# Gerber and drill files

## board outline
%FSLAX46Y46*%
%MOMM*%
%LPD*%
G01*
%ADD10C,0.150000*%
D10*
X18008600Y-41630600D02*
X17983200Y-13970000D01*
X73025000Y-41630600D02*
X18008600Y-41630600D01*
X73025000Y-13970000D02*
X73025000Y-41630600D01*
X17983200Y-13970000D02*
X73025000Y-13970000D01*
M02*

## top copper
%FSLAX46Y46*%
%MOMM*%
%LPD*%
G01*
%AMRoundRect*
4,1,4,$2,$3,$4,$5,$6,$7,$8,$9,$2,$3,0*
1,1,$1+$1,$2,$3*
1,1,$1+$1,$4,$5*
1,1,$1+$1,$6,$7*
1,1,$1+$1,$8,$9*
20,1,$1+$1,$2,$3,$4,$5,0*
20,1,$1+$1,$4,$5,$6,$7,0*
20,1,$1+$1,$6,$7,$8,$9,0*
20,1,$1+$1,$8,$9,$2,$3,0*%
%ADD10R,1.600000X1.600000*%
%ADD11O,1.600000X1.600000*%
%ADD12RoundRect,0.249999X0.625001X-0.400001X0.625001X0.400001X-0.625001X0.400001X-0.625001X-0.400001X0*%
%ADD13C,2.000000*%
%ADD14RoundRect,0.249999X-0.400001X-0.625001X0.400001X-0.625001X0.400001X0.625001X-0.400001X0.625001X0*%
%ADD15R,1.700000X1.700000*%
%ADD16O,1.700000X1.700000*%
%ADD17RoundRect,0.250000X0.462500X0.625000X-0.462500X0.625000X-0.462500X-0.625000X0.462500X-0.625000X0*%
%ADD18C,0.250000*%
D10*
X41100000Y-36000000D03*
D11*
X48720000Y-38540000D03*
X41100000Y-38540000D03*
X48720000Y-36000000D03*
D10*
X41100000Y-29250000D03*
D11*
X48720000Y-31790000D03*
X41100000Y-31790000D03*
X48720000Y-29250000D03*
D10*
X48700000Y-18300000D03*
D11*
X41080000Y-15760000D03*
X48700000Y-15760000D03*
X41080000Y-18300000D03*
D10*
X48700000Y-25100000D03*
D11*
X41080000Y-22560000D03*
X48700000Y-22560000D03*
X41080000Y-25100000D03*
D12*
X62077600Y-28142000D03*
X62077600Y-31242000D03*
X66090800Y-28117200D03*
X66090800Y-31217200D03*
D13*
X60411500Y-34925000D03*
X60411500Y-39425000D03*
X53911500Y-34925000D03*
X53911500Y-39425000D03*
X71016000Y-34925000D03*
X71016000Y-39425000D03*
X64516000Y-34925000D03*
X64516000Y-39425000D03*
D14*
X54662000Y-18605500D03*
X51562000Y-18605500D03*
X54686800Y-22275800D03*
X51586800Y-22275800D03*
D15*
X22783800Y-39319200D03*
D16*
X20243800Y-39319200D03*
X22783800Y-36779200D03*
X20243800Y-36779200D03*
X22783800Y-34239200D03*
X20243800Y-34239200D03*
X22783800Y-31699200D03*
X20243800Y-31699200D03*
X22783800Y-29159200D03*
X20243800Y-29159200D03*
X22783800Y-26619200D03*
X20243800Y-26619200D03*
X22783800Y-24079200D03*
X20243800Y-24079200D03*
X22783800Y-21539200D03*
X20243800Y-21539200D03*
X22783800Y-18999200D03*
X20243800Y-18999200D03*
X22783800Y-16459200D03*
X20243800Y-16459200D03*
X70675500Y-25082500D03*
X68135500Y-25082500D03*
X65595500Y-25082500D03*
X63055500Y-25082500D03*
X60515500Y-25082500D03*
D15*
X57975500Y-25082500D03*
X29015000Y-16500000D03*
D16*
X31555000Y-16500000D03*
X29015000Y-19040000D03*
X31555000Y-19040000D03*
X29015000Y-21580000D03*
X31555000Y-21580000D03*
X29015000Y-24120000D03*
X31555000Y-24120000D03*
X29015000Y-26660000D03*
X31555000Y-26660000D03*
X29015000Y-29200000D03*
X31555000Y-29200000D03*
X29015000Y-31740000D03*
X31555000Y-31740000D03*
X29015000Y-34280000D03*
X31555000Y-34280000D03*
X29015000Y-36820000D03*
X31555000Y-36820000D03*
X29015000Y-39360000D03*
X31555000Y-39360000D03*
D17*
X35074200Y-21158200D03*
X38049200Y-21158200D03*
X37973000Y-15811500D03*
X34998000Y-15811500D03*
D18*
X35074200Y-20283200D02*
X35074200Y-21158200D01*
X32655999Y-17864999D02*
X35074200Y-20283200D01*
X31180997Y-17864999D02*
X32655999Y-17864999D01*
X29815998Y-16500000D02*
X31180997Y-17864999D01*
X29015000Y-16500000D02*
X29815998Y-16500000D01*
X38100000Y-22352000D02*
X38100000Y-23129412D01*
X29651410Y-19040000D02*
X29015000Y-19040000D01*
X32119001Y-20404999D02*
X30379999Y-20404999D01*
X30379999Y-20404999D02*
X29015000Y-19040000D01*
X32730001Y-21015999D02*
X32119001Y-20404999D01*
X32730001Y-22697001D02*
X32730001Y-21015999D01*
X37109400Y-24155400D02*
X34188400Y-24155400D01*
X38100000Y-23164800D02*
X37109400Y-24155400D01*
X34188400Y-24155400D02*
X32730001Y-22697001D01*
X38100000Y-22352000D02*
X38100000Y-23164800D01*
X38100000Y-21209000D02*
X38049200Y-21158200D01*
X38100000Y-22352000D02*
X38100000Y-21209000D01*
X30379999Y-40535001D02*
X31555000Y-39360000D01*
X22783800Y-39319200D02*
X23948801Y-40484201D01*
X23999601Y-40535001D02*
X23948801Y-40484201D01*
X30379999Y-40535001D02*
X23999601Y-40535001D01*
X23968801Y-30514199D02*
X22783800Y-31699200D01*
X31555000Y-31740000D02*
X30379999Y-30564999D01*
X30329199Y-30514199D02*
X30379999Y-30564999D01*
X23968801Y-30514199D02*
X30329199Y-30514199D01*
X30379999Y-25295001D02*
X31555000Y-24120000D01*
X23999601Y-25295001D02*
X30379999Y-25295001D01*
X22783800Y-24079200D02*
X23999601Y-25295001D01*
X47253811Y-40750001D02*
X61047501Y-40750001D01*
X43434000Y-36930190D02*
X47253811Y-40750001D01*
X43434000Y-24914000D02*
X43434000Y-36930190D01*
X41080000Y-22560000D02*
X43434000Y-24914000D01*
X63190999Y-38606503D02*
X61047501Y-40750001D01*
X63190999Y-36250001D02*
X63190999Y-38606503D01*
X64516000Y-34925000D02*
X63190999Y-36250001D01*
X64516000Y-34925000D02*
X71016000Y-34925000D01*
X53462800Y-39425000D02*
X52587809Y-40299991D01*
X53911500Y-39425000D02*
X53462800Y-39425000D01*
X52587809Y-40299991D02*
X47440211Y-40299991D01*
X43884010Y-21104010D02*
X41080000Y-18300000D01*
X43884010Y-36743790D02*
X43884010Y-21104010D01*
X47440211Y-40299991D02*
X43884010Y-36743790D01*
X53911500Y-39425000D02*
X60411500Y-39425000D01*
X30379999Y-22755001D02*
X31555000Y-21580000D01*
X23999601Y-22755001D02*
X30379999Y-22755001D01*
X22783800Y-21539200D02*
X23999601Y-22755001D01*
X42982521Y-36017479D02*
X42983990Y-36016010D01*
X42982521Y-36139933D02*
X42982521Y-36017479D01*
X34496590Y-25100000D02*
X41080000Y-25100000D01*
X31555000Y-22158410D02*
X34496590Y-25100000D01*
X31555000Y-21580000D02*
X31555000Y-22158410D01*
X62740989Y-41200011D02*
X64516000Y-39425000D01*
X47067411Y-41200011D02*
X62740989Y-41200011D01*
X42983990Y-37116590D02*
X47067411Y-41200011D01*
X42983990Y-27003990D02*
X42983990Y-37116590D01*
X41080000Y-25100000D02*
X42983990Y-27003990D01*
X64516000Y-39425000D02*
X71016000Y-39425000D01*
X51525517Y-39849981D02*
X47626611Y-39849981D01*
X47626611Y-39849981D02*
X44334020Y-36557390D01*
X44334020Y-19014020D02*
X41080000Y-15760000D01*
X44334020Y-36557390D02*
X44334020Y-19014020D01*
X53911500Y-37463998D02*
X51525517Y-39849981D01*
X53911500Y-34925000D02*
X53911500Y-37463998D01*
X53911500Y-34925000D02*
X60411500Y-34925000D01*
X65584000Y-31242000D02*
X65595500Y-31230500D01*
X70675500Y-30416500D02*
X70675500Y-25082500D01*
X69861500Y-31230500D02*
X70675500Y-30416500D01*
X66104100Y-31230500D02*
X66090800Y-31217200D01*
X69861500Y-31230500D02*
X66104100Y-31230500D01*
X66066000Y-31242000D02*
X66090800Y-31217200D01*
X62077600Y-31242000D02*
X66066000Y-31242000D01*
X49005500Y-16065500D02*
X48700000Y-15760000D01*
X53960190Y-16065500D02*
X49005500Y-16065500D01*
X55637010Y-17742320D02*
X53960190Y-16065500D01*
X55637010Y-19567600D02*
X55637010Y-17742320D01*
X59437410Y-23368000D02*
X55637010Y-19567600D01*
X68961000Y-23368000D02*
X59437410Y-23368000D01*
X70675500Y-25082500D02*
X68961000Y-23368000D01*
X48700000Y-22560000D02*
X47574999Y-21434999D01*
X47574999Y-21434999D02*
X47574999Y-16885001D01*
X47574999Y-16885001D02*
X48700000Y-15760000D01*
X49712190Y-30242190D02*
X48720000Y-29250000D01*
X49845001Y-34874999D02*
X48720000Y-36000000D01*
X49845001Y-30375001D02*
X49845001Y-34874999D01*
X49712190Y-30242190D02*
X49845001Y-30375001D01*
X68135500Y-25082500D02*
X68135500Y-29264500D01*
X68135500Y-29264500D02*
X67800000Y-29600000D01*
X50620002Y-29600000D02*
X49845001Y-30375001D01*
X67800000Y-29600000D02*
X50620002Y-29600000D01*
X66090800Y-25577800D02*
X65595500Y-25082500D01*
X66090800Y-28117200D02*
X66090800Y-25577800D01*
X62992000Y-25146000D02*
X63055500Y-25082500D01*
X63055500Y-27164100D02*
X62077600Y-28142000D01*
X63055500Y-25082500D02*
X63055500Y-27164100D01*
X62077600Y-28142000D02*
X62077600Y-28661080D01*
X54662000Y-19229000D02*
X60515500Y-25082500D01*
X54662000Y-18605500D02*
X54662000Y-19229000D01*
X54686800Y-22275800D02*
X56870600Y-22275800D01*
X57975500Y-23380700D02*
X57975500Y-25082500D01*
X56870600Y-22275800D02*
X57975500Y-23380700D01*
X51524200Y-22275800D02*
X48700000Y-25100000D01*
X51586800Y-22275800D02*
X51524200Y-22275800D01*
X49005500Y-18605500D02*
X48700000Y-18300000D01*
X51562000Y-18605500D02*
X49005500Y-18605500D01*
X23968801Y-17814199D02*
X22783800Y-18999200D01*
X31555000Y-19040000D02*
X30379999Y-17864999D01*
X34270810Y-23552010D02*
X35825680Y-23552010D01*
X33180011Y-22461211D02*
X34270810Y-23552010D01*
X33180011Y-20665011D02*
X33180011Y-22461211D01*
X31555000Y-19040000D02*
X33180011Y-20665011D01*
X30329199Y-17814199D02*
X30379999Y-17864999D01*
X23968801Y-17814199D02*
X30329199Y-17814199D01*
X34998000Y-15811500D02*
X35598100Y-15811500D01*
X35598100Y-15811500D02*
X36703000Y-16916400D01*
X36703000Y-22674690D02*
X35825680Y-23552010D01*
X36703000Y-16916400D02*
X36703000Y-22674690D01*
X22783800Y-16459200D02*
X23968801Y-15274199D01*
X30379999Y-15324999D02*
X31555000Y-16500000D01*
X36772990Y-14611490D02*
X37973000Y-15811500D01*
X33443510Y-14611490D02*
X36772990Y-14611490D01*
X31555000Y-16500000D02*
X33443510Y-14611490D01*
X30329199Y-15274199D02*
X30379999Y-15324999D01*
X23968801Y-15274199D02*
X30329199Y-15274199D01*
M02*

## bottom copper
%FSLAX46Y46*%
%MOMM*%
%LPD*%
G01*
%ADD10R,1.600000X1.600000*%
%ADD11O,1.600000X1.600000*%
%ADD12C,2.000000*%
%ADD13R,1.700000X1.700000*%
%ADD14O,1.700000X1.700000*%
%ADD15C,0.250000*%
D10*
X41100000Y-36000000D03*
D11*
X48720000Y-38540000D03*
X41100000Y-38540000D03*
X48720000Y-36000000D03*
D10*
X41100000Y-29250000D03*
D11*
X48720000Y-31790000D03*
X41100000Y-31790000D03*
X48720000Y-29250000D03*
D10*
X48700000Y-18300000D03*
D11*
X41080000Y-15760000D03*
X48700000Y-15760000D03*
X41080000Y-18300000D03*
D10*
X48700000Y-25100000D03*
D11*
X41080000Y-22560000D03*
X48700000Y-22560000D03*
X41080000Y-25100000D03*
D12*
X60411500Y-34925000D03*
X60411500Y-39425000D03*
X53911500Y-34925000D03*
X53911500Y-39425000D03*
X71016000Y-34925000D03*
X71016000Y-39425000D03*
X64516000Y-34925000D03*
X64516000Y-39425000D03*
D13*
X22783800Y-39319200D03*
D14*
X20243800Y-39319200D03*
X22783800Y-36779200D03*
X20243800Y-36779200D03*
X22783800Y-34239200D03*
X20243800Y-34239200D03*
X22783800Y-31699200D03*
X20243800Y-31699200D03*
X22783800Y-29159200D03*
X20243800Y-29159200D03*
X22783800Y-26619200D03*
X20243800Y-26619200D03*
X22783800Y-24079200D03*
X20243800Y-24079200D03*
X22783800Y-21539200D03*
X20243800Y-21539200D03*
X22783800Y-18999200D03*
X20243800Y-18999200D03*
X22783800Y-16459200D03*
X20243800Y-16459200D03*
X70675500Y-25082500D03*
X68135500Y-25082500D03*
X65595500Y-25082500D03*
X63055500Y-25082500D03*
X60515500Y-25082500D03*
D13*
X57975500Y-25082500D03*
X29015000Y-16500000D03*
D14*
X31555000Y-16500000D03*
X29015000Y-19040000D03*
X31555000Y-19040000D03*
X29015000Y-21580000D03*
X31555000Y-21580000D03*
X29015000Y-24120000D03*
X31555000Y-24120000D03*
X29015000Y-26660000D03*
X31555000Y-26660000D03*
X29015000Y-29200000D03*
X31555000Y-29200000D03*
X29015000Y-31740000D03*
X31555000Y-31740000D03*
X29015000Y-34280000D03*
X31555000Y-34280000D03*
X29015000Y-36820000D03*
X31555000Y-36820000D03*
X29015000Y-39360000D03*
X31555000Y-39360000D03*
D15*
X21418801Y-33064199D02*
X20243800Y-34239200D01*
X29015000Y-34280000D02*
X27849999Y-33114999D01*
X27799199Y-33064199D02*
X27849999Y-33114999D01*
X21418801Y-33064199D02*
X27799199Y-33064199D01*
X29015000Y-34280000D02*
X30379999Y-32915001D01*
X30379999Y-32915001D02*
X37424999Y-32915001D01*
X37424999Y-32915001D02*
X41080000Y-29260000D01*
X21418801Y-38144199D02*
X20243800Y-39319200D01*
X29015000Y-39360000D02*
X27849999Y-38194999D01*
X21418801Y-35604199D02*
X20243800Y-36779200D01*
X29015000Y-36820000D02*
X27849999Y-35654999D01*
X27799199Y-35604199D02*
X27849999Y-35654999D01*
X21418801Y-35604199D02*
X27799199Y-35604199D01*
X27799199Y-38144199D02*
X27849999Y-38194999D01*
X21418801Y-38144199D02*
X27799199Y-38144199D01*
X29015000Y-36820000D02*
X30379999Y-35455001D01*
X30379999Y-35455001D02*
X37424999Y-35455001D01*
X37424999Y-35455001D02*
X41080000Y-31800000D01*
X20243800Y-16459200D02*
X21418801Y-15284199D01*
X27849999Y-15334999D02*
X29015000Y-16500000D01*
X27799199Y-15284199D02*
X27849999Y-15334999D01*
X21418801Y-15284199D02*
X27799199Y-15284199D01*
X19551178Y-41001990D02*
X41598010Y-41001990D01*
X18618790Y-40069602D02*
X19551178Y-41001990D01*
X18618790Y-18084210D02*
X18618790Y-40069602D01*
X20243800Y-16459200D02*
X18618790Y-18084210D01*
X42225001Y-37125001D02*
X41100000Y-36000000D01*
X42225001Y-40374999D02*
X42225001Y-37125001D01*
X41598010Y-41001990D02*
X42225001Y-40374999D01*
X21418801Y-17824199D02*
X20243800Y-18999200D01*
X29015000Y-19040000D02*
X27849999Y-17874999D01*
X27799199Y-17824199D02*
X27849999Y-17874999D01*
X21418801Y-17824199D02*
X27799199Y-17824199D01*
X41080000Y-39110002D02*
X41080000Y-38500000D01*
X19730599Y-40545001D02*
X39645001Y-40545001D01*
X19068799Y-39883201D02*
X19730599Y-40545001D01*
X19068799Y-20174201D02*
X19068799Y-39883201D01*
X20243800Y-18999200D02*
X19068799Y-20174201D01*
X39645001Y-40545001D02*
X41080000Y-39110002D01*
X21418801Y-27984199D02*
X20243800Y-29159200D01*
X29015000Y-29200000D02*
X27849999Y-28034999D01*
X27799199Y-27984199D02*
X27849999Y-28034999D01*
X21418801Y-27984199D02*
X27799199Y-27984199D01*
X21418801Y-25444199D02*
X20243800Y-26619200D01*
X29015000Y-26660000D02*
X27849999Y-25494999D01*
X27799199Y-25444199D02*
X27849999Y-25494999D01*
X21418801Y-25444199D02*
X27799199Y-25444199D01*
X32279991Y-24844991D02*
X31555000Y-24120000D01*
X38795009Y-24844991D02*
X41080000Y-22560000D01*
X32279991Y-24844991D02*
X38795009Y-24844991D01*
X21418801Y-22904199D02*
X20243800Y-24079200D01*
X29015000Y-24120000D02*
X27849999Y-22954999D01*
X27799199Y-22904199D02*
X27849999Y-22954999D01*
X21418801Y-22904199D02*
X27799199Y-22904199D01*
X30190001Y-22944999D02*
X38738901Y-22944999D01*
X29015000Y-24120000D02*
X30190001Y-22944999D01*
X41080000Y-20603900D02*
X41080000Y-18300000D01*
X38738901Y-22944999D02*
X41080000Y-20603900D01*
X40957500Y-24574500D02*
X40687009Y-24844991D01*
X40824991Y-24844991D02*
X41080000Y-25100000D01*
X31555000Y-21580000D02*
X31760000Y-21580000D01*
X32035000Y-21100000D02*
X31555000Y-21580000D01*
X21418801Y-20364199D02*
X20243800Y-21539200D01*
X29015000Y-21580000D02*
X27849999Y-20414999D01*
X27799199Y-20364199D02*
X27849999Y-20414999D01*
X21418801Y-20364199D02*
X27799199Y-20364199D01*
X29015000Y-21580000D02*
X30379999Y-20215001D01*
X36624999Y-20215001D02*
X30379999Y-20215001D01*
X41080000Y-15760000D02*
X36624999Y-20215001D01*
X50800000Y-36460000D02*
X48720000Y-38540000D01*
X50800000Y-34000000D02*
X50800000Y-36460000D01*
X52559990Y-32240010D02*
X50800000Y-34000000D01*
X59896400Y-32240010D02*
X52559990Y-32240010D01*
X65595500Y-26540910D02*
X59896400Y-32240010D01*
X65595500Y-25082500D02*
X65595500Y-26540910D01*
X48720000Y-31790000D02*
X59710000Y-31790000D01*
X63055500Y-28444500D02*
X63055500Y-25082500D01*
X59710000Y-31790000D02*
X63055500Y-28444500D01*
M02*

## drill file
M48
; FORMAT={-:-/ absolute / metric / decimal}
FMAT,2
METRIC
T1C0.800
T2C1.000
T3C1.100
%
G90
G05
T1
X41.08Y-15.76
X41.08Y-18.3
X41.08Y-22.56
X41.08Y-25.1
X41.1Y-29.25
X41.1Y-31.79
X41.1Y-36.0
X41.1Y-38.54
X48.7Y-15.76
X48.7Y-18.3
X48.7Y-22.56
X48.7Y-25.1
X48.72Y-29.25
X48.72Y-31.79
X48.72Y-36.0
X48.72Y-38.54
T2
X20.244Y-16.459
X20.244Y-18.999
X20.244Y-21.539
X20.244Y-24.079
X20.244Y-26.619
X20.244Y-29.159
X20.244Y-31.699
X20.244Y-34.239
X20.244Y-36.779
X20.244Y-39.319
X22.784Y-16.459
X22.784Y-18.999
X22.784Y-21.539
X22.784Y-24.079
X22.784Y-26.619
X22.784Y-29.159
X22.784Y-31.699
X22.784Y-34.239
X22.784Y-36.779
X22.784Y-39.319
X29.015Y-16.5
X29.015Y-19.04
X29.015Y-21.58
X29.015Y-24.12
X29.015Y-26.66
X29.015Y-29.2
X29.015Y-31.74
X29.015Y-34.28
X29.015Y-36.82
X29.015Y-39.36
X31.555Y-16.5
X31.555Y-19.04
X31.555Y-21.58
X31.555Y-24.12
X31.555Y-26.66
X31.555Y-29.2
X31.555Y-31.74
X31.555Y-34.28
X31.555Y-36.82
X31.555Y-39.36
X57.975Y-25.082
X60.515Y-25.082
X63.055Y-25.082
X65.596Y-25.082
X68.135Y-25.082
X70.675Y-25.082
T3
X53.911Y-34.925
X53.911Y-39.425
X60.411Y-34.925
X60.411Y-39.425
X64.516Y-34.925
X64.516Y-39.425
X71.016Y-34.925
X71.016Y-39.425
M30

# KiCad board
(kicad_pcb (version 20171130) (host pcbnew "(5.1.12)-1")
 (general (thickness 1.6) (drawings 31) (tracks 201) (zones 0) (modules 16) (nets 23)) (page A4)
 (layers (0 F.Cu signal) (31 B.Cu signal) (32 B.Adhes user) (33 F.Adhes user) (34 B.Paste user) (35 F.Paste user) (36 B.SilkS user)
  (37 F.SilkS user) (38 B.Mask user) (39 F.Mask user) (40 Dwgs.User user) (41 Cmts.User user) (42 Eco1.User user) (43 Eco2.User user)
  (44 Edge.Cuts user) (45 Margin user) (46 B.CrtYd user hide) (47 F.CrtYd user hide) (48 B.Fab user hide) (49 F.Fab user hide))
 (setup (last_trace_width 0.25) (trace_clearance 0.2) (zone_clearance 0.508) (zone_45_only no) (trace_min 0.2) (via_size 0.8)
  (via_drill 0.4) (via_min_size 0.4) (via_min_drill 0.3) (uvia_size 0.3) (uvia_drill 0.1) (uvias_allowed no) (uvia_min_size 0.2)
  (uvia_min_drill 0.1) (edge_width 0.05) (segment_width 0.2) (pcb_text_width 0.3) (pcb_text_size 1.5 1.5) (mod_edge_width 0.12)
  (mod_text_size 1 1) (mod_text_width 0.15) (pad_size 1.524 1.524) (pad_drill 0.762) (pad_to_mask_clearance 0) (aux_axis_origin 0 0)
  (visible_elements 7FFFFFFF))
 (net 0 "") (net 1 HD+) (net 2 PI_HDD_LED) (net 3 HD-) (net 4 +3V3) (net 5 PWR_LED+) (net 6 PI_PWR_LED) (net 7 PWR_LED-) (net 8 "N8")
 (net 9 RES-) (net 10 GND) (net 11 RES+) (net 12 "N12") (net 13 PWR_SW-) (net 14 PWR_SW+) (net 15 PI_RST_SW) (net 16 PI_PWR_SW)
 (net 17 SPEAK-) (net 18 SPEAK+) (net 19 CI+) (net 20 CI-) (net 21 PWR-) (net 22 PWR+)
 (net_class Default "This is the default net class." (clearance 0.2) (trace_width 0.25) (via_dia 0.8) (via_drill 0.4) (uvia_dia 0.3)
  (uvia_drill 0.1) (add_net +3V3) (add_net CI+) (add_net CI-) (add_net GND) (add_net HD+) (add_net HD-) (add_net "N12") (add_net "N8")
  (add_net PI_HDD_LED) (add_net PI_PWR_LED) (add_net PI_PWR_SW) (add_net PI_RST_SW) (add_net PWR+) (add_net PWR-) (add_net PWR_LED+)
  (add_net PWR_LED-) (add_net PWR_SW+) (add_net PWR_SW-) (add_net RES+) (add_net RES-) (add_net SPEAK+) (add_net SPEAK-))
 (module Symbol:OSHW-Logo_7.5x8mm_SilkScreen (layer F.Cu) (at 54.4 29.5 270)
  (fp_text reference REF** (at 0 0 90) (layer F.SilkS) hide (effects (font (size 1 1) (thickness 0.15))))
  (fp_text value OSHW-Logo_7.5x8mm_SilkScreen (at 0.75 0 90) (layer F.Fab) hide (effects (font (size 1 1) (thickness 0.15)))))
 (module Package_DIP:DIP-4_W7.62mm (layer F.Cu) (at 41.1 36)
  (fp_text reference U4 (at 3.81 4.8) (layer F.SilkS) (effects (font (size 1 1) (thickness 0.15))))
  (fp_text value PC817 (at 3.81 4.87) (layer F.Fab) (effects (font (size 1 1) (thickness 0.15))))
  (pad 1 thru_hole rect (at 0 0) (size 1.6 1.6) (drill 0.8) (layers *.Cu *.Mask) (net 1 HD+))
  (pad 3 thru_hole oval (at 7.62 2.54) (size 1.6 1.6) (drill 0.8) (layers *.Cu *.Mask) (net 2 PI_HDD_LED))
  (pad 2 thru_hole oval (at 0 2.54) (size 1.6 1.6) (drill 0.8) (layers *.Cu *.Mask) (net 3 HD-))
  (pad 4 thru_hole oval (at 7.62 0) (size 1.6 1.6) (drill 0.8) (layers *.Cu *.Mask) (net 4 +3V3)))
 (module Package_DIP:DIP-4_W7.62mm (layer F.Cu) (at 41.1 29.25)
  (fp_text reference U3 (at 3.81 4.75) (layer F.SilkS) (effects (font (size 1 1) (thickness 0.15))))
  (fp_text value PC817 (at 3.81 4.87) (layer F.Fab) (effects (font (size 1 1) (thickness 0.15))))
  (pad 1 thru_hole rect (at 0 0) (size 1.6 1.6) (drill 0.8) (layers *.Cu *.Mask) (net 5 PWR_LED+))
  (pad 3 thru_hole oval (at 7.62 2.54) (size 1.6 1.6) (drill 0.8) (layers *.Cu *.Mask) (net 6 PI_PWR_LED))
  (pad 2 thru_hole oval (at 0 2.54) (size 1.6 1.6) (drill 0.8) (layers *.Cu *.Mask) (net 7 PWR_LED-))
  (pad 4 thru_hole oval (at 7.62 0) (size 1.6 1.6) (drill 0.8) (layers *.Cu *.Mask) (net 4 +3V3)))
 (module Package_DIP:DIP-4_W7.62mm (layer F.Cu) (at 48.7 18.3 180)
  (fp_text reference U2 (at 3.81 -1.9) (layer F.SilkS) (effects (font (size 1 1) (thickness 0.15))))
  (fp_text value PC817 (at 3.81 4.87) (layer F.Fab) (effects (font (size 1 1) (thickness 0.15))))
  (pad 1 thru_hole rect (at 0 0 180) (size 1.6 1.6) (drill 0.8) (layers *.Cu *.Mask) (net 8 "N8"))
  (pad 3 thru_hole oval (at 7.62 2.54 180) (size 1.6 1.6) (drill 0.8) (layers *.Cu *.Mask) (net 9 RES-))
  (pad 2 thru_hole oval (at 0 2.54 180) (size 1.6 1.6) (drill 0.8) (layers *.Cu *.Mask) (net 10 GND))
  (pad 4 thru_hole oval (at 7.62 0 180) (size 1.6 1.6) (drill 0.8) (layers *.Cu *.Mask) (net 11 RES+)))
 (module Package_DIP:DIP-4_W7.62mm (layer F.Cu) (at 48.7 25.1 180)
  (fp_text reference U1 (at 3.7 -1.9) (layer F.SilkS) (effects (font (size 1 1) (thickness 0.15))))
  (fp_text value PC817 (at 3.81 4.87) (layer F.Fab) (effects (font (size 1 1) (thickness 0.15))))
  (pad 1 thru_hole rect (at 0 0 180) (size 1.6 1.6) (drill 0.8) (layers *.Cu *.Mask) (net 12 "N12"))
  (pad 3 thru_hole oval (at 7.62 2.54 180) (size 1.6 1.6) (drill 0.8) (layers *.Cu *.Mask) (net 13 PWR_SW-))
  (pad 2 thru_hole oval (at 0 2.54 180) (size 1.6 1.6) (drill 0.8) (layers *.Cu *.Mask) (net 10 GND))
  (pad 4 thru_hole oval (at 7.62 0 180) (size 1.6 1.6) (drill 0.8) (layers *.Cu *.Mask) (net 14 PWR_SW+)))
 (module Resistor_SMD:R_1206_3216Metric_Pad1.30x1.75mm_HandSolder (layer F.Cu) (at 62.0776 29.692 90)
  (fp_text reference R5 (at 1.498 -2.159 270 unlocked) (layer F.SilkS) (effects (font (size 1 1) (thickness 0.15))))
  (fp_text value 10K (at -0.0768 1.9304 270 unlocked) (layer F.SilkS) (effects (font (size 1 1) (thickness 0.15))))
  (pad 2 smd roundrect (at 1.55 0 90) (size 1.3 1.75) (layers F.Cu F.Paste F.Mask) (roundrect_rratio 0.1923069230769231) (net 6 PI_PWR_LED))
  (pad 1 smd roundrect (at -1.55 0 90) (size 1.3 1.75) (layers F.Cu F.Paste F.Mask) (roundrect_rratio 0.1923069230769231) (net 10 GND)))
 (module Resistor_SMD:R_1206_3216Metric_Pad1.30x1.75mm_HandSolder (layer F.Cu) (at 66.0908 29.6672 90)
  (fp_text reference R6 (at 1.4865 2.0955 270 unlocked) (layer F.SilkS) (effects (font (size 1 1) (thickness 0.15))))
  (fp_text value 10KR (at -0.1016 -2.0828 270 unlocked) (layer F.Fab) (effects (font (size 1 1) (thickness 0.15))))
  (pad 2 smd roundrect (at 1.55 0 90) (size 1.3 1.75) (layers F.Cu F.Paste F.Mask) (roundrect_rratio 0.1923069230769231) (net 2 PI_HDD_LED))
  (pad 1 smd roundrect (at -1.55 0 90) (size 1.3 1.75) (layers F.Cu F.Paste F.Mask) (roundrect_rratio 0.1923069230769231) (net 10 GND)))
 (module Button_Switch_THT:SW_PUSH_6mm (layer F.Cu) (at 53.9115 34.925)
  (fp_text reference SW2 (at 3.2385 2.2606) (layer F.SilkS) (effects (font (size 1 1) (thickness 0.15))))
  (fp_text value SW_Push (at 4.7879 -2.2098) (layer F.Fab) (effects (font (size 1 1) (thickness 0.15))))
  (pad 1 thru_hole circle (at 6.5 0 90) (size 2 2) (drill 1.1) (layers *.Cu *.Mask) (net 9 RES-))
  (pad 2 thru_hole circle (at 6.5 4.5 90) (size 2 2) (drill 1.1) (layers *.Cu *.Mask) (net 11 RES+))
  (pad 1 thru_hole circle (at 0 0 90) (size 2 2) (drill 1.1) (layers *.Cu *.Mask) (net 9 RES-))
  (pad 2 thru_hole circle (at 0 4.5 90) (size 2 2) (drill 1.1) (layers *.Cu *.Mask) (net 11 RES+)))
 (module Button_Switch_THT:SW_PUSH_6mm (layer F.Cu) (at 64.516 34.925)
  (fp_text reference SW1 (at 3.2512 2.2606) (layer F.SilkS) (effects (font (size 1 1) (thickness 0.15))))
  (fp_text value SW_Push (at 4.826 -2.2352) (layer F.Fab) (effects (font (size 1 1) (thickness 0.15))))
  (pad 1 thru_hole circle (at 6.5 0 90) (size 2 2) (drill 1.1) (layers *.Cu *.Mask) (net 13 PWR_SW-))
  (pad 2 thru_hole circle (at 6.5 4.5 90) (size 2 2) (drill 1.1) (layers *.Cu *.Mask) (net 14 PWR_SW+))
  (pad 1 thru_hole circle (at 0 0 90) (size 2 2) (drill 1.1) (layers *.Cu *.Mask) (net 13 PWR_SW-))
  (pad 2 thru_hole circle (at 0 4.5 90) (size 2 2) (drill 1.1) (layers *.Cu *.Mask) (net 14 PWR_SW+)))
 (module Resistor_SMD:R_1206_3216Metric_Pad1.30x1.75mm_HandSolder (layer F.Cu) (at 53.112 18.6055)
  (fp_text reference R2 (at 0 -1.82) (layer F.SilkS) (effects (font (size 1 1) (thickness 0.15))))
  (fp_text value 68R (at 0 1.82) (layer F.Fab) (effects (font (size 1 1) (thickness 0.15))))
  (pad 2 smd roundrect (at 1.55 0) (size 1.3 1.75) (layers F.Cu F.Paste F.Mask) (roundrect_rratio 0.1923069230769231) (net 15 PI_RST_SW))
  (pad 1 smd roundrect (at -1.55 0) (size 1.3 1.75) (layers F.Cu F.Paste F.Mask) (roundrect_rratio 0.1923069230769231) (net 8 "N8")))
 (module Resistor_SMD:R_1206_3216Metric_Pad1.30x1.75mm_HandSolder (layer F.Cu) (at 53.1368 22.2758)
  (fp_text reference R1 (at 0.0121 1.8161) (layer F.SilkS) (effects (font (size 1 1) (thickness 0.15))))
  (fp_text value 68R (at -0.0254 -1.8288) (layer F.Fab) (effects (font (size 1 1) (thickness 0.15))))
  (pad 2 smd roundrect (at 1.55 0) (size 1.3 1.75) (layers F.Cu F.Paste F.Mask) (roundrect_rratio 0.1923069230769231) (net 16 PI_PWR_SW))
  (pad 1 smd roundrect (at -1.55 0) (size 1.3 1.75) (layers F.Cu F.Paste F.Mask) (roundrect_rratio 0.1923069230769231) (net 12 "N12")))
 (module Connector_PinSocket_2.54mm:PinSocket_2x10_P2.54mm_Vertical (layer B.Cu) (at 22.7838 39.3192)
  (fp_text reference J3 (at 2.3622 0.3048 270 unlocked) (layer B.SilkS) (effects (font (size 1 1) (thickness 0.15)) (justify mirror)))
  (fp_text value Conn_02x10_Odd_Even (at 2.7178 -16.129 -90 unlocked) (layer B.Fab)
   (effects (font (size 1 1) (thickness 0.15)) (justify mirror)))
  (pad 1 thru_hole rect (at 0 0) (size 1.7 1.7) (drill 1) (layers *.Cu *.Mask) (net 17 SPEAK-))
  (pad 2 thru_hole oval (at -2.54 0) (size 1.7 1.7) (drill 1) (layers *.Cu *.Mask) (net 7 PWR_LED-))
  (pad 3 thru_hole oval (at 0 -2.54) (size 1.7 1.7) (drill 1) (layers *.Cu *.Mask))
  (pad 4 thru_hole oval (at -2.54 -2.54) (size 1.7 1.7) (drill 1) (layers *.Cu *.Mask) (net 7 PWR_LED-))
  (pad 5 thru_hole oval (at 0 -5.08) (size 1.7 1.7) (drill 1) (layers *.Cu *.Mask))
  (pad 6 thru_hole oval (at -2.54 -5.08) (size 1.7 1.7) (drill 1) (layers *.Cu *.Mask) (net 5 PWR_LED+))
  (pad 7 thru_hole oval (at 0 -7.62) (size 1.7 1.7) (drill 1) (layers *.Cu *.Mask) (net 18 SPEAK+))
  (pad 8 thru_hole oval (at -2.54 -7.62) (size 1.7 1.7) (drill 1) (layers *.Cu *.Mask))
  (pad 9 thru_hole oval (at 0 -10.16) (size 1.7 1.7) (drill 1) (layers *.Cu *.Mask))
  (pad 10 thru_hole oval (at -2.54 -10.16) (size 1.7 1.7) (drill 1) (layers *.Cu *.Mask) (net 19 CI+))
  (pad 11 thru_hole oval (at 0 -12.7) (size 1.7 1.7) (drill 1) (layers *.Cu *.Mask))
  (pad 12 thru_hole oval (at -2.54 -12.7) (size 1.7 1.7) (drill 1) (layers *.Cu *.Mask) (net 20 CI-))
  (pad 13 thru_hole oval (at 0 -15.24) (size 1.7 1.7) (drill 1) (layers *.Cu *.Mask) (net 13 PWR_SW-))
  (pad 14 thru_hole oval (at -2.54 -15.24) (size 1.7 1.7) (drill 1) (layers *.Cu *.Mask) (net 11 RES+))
  (pad 15 thru_hole oval (at 0 -17.78) (size 1.7 1.7) (drill 1) (layers *.Cu *.Mask) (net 14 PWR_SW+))
  (pad 16 thru_hole oval (at -2.54 -17.78) (size 1.7 1.7) (drill 1) (layers *.Cu *.Mask) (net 9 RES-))
  (pad 17 thru_hole oval (at 0 -20.32) (size 1.7 1.7) (drill 1) (layers *.Cu *.Mask) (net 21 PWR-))
  (pad 18 thru_hole oval (at -2.54 -20.32) (size 1.7 1.7) (drill 1) (layers *.Cu *.Mask) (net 3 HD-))
  (pad 19 thru_hole oval (at 0 -22.86) (size 1.7 1.7) (drill 1) (layers *.Cu *.Mask) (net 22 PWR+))
  (pad 20 thru_hole oval (at -2.54 -22.86) (size 1.7 1.7) (drill 1) (layers *.Cu *.Mask) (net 1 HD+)))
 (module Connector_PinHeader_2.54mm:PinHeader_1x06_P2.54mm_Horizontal (layer F.Cu) (at 57.9755 25.0825 90)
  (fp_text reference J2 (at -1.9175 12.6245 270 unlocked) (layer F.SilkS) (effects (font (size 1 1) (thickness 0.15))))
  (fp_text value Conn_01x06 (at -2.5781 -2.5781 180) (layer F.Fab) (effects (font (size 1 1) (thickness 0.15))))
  (pad 6 thru_hole oval (at 0 12.7 90) (size 1.7 1.7) (drill 1) (layers *.Cu *.Mask) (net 10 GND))
  (pad 5 thru_hole oval (at 0 10.16 90) (size 1.7 1.7) (drill 1) (layers *.Cu *.Mask) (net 4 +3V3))
  (pad 4 thru_hole oval (at 0 7.62 90) (size 1.7 1.7) (drill 1) (layers *.Cu *.Mask) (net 2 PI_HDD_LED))
  (pad 3 thru_hole oval (at 0 5.08 90) (size 1.7 1.7) (drill 1) (layers *.Cu *.Mask) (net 6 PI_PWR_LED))
  (pad 2 thru_hole oval (at 0 2.54 90) (size 1.7 1.7) (drill 1) (layers *.Cu *.Mask) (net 15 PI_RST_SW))
  (pad 1 thru_hole rect (at 0 0 90) (size 1.7 1.7) (drill 1) (layers *.Cu *.Mask) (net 16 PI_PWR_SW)))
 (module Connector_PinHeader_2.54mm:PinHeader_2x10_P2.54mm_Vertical (layer F.Cu) (at 29.015 16.5)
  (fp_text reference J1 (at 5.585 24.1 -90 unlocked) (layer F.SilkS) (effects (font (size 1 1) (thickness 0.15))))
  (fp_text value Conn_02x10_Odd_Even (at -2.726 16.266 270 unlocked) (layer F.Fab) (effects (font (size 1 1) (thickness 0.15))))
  (pad 1 thru_hole rect (at 0 0) (size 1.7 1.7) (drill 1) (layers *.Cu *.Mask) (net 1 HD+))
  (pad 2 thru_hole oval (at 2.54 0) (size 1.7 1.7) (drill 1) (layers *.Cu *.Mask) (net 22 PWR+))
  (pad 3 thru_hole oval (at 0 2.54) (size 1.7 1.7) (drill 1) (layers *.Cu *.Mask) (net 3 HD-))
  (pad 4 thru_hole oval (at 2.54 2.54) (size 1.7 1.7) (drill 1) (layers *.Cu *.Mask) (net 21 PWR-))
  (pad 5 thru_hole oval (at 0 5.08) (size 1.7 1.7) (drill 1) (layers *.Cu *.Mask) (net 9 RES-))
  (pad 6 thru_hole oval (at 2.54 5.08) (size 1.7 1.7) (drill 1) (layers *.Cu *.Mask) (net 14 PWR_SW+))
  (pad 7 thru_hole oval (at 0 7.62) (size 1.7 1.7) (drill 1) (layers *.Cu *.Mask) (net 11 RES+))
  (pad 8 thru_hole oval (at 2.54 7.62) (size 1.7 1.7) (drill 1) (layers *.Cu *.Mask) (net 13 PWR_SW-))
  (pad 9 thru_hole oval (at 0 10.16) (size 1.7 1.7) (drill 1) (layers *.Cu *.Mask) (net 20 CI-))
  (pad 10 thru_hole oval (at 2.54 10.16) (size 1.7 1.7) (drill 1) (layers *.Cu *.Mask))
  (pad 11 thru_hole oval (at 0 12.7) (size 1.7 1.7) (drill 1) (layers *.Cu *.Mask) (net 19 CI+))
  (pad 12 thru_hole oval (at 2.54 12.7) (size 1.7 1.7) (drill 1) (layers *.Cu *.Mask))
  (pad 13 thru_hole oval (at 0 15.24) (size 1.7 1.7) (drill 1) (layers *.Cu *.Mask))
  (pad 14 thru_hole oval (at 2.54 15.24) (size 1.7 1.7) (drill 1) (layers *.Cu *.Mask) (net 18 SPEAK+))
  (pad 15 thru_hole oval (at 0 17.78) (size 1.7 1.7) (drill 1) (layers *.Cu *.Mask) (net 5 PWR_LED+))
  (pad 16 thru_hole oval (at 2.54 17.78) (size 1.7 1.7) (drill 1) (layers *.Cu *.Mask))
  (pad 17 thru_hole oval (at 0 20.32) (size 1.7 1.7) (drill 1) (layers *.Cu *.Mask) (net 7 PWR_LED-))
  (pad 18 thru_hole oval (at 2.54 20.32) (size 1.7 1.7) (drill 1) (layers *.Cu *.Mask))
  (pad 19 thru_hole oval (at 0 22.86) (size 1.7 1.7) (drill 1) (layers *.Cu *.Mask) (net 7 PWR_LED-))
  (pad 20 thru_hole oval (at 2.54 22.86) (size 1.7 1.7) (drill 1) (layers *.Cu *.Mask) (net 17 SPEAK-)))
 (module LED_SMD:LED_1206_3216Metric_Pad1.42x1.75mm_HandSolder (layer F.Cu) (at 36.5617 21.1582 180)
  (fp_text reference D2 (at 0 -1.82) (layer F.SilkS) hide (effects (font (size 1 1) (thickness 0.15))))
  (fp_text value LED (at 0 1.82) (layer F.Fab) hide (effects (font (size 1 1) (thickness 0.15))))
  (pad 2 smd roundrect (at 1.4875 0 180) (size 1.425 1.75) (layers F.Cu F.Paste F.Mask) (roundrect_rratio 0.1754385964912281) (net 1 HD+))
  (pad 1 smd roundrect (at -1.4875 0 180) (size 1.425 1.75) (layers F.Cu F.Paste F.Mask) (roundrect_rratio 0.1754385964912281) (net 3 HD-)))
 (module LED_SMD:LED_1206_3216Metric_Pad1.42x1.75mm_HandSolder (layer F.Cu) (at 36.4855 15.8115 180)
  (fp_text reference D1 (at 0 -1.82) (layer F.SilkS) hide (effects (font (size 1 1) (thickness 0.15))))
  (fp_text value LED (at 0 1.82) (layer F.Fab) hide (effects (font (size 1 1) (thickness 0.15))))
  (pad 1 smd roundrect (at -1.4875 0 180) (size 1.425 1.75) (layers F.Cu F.Paste F.Mask) (roundrect_rratio 0.1754385964912281) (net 22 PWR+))
  (pad 2 smd roundrect (at 1.4875 0 180) (size 1.425 1.75) (layers F.Cu F.Paste F.Mask) (roundrect_rratio 0.1754385964912281) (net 21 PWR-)))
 (gr_line (start 18.0086 41.6306) (end 17.9832 13.97) (layer Edge.Cuts) (width 0.15))
 (gr_line (start 73.025 41.6306) (end 18.0086 41.6306) (layer Edge.Cuts) (width 0.15))
 (gr_line (start 73.025 13.97) (end 73.025 41.6306) (layer Edge.Cuts) (width 0.15))
 (gr_line (start 17.9832 13.97) (end 73.025 13.97) (layer Edge.Cuts) (width 0.15))
 (segment (start 21.418801 33.064199) (end 20.2438 34.2392) (width 0.25) (layer B.Cu) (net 5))
 (segment (start 29.015 34.28) (end 27.849999 33.114999) (width 0.25) (layer B.Cu) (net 5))
 (segment (start 27.799199 33.064199) (end 27.849999 33.114999) (width 0.25) (layer B.Cu) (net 5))
 (segment (start 21.418801 33.064199) (end 27.799199 33.064199) (width 0.25) (layer B.Cu) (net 5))
 (segment (start 29.015 34.28) (end 30.379999 32.915001) (width 0.25) (layer B.Cu) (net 5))
 (segment (start 30.379999 32.915001) (end 37.424999 32.915001) (width 0.25) (layer B.Cu) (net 5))
 (segment (start 37.424999 32.915001) (end 41.08 29.26) (width 0.25) (layer B.Cu) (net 5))
 (segment (start 21.418801 38.144199) (end 20.2438 39.3192) (width 0.25) (layer B.Cu) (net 7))
 (segment (start 29.015 39.36) (end 27.849999 38.194999) (width 0.25) (layer B.Cu) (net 7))
 (segment (start 21.418801 35.604199) (end 20.2438 36.7792) (width 0.25) (layer B.Cu) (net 7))
 (segment (start 29.015 36.82) (end 27.849999 35.654999) (width 0.25) (layer B.Cu) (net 7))
 (segment (start 27.799199 35.604199) (end 27.849999 35.654999) (width 0.25) (layer B.Cu) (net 7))
 (segment (start 21.418801 35.604199) (end 27.799199 35.604199) (width 0.25) (layer B.Cu) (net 7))
 (segment (start 27.799199 38.144199) (end 27.849999 38.194999) (width 0.25) (layer B.Cu) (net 7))
 (segment (start 21.418801 38.144199) (end 27.799199 38.144199) (width 0.25) (layer B.Cu) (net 7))
 (segment (start 29.015 36.82) (end 30.379999 35.455001) (width 0.25) (layer B.Cu) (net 7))
 (segment (start 30.379999 35.455001) (end 37.424999 35.455001) (width 0.25) (layer B.Cu) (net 7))
 (segment (start 37.424999 35.455001) (end 41.08 31.8) (width 0.25) (layer B.Cu) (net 7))
 (segment (start 20.2438 16.4592) (end 21.418801 15.284199) (width 0.25) (layer B.Cu) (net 1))
 (segment (start 27.849999 15.334999) (end 29.015 16.5) (width 0.25) (layer B.Cu) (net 1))
 (segment (start 27.799199 15.284199) (end 27.849999 15.334999) (width 0.25) (layer B.Cu) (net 1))
 (segment (start 21.418801 15.284199) (end 27.799199 15.284199) (width 0.25) (layer B.Cu) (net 1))
 (segment (start 35.0742 20.2832) (end 35.0742 21.1582) (width 0.25) (layer F.Cu) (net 1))
 (segment (start 32.655999 17.864999) (end 35.0742 20.2832) (width 0.25) (layer F.Cu) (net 1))
 (segment (start 31.180997 17.864999) (end 32.655999 17.864999) (width 0.25) (layer F.Cu) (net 1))
 (segment (start 29.815998 16.5) (end 31.180997 17.864999) (width 0.25) (layer F.Cu) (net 1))
 (segment (start 29.015 16.5) (end 29.815998 16.5) (width 0.25) (layer F.Cu) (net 1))
 (segment (start 19.551178 41.00199) (end 41.59801 41.00199) (width 0.25) (layer B.Cu) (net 1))
 (segment (start 18.61879 40.069602) (end 19.551178 41.00199) (width 0.25) (layer B.Cu) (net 1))
 (segment (start 18.61879 18.08421) (end 18.61879 40.069602) (width 0.25) (layer B.Cu) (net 1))
 (segment (start 20.2438 16.4592) (end 18.61879 18.08421) (width 0.25) (layer B.Cu) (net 1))
 (segment (start 42.225001 37.125001) (end 41.1 36) (width 0.25) (layer B.Cu) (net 1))
 (segment (start 42.225001 40.374999) (end 42.225001 37.125001) (width 0.25) (layer B.Cu) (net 1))
 (segment (start 41.59801 41.00199) (end 42.225001 40.374999) (width 0.25) (layer B.Cu) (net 1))
 (segment (start 38.1 22.352) (end 38.1 23.129412) (width 0.25) (layer F.Cu) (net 3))
 (segment (start 21.418801 17.824199) (end 20.2438 18.9992) (width 0.25) (layer B.Cu) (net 3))
 (segment (start 29.015 19.04) (end 27.849999 17.874999) (width 0.25) (layer B.Cu) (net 3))
 (segment (start 29.65141 19.04) (end 29.015 19.04) (width 0.25) (layer F.Cu) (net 3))
 (segment (start 32.119001 20.404999) (end 30.379999 20.404999) (width 0.25) (layer F.Cu) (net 3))
 (segment (start 30.379999 20.404999) (end 29.015 19.04) (width 0.25) (layer F.Cu) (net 3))
 (segment (start 32.730001 21.015999) (end 32.119001 20.404999) (width 0.25) (layer F.Cu) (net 3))
 (segment (start 32.730001 22.697001) (end 32.730001 21.015999) (width 0.25) (layer F.Cu) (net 3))
 (segment (start 37.1094 24.1554) (end 34.1884 24.1554) (width 0.25) (layer F.Cu) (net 3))
 (segment (start 38.1 23.1648) (end 37.1094 24.1554) (width 0.25) (layer F.Cu) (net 3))
 (segment (start 34.1884 24.1554) (end 32.730001 22.697001) (width 0.25) (layer F.Cu) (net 3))
 (segment (start 38.1 22.352) (end 38.1 23.1648) (width 0.25) (layer F.Cu) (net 3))
 (segment (start 27.799199 17.824199) (end 27.849999 17.874999) (width 0.25) (layer B.Cu) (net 3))
 (segment (start 21.418801 17.824199) (end 27.799199 17.824199) (width 0.25) (layer B.Cu) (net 3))
 (segment (start 38.1 21.209) (end 38.0492 21.1582) (width 0.25) (layer F.Cu) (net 3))
 (segment (start 38.1 22.352) (end 38.1 21.209) (width 0.25) (layer F.Cu) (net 3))
 (segment (start 41.08 39.110002) (end 41.08 38.5) (width 0.25) (layer B.Cu) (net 3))
 (segment (start 19.730599 40.545001) (end 39.645001 40.545001) (width 0.25) (layer B.Cu) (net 3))
 (segment (start 19.068799 39.883201) (end 19.730599 40.545001) (width 0.25) (layer B.Cu) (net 3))
 (segment (start 19.068799 20.174201) (end 19.068799 39.883201) (width 0.25) (layer B.Cu) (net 3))
 (segment (start 20.2438 18.9992) (end 19.068799 20.174201) (width 0.25) (layer B.Cu) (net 3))
 (segment (start 39.645001 40.545001) (end 41.08 39.110002) (width 0.25) (layer B.Cu) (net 3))
 (segment (start 30.379999 40.535001) (end 31.555 39.36) (width 0.25) (layer F.Cu) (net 17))
 (segment (start 22.7838 39.3192) (end 23.948801 40.484201) (width 0.25) (layer F.Cu) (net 17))
 (segment (start 23.999601 40.535001) (end 23.948801 40.484201) (width 0.25) (layer F.Cu) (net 17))
 (segment (start 30.379999 40.535001) (end 23.999601 40.535001) (width 0.25) (layer F.Cu) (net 17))
 (segment (start 23.968801 30.514199) (end 22.7838 31.6992) (width 0.25) (layer F.Cu) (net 18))
 (segment (start 31.555 31.74) (end 30.379999 30.564999) (width 0.25) (layer F.Cu) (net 18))
 (segment (start 30.329199 30.514199) (end 30.379999 30.564999) (width 0.25) (layer F.Cu) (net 18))
 (segment (start 23.968801 30.514199) (end 30.329199 30.514199) (width 0.25) (layer F.Cu) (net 18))
 (segment (start 21.418801 27.984199) (end 20.2438 29.1592) (width 0.25) (layer B.Cu) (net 19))
 (segment (start 29.015 29.2) (end 27.849999 28.034999) (width 0.25) (layer B.Cu) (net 19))
 (segment (start 27.799199 27.984199) (end 27.849999 28.034999) (width 0.25) (layer B.Cu) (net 19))
 (segment (start 21.418801 27.984199) (end 27.799199 27.984199) (width 0.25) (layer B.Cu) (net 19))
 (segment (start 21.418801 25.444199) (end 20.2438 26.6192) (width 0.25) (layer B.Cu) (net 20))
 (segment (start 29.015 26.66) (end 27.849999 25.494999) (width 0.25) (layer B.Cu) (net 20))
 (segment (start 27.799199 25.444199) (end 27.849999 25.494999) (width 0.25) (layer B.Cu) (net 20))
 (segment (start 21.418801 25.444199) (end 27.799199 25.444199) (width 0.25) (layer B.Cu) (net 20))
 (segment (start 32.279991 24.844991) (end 31.555 24.12) (width 0.25) (layer B.Cu) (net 13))
 (segment (start 30.379999 25.295001) (end 31.555 24.12) (width 0.25) (layer F.Cu) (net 13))
 (segment (start 23.999601 25.295001) (end 30.379999 25.295001) (width 0.25) (layer F.Cu) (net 13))
 (segment (start 22.7838 24.0792) (end 23.999601 25.295001) (width 0.25) (layer F.Cu) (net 13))
 (segment (start 38.795009 24.844991) (end 41.08 22.56) (width 0.25) (layer B.Cu) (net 13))
 (segment (start 32.279991 24.844991) (end 38.795009 24.844991) (width 0.25) (layer B.Cu) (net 13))
 (segment (start 47.253811 40.750001) (end 61.047501 40.750001) (width 0.25) (layer F.Cu) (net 13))
 (segment (start 43.434 36.93019) (end 47.253811 40.750001) (width 0.25) (layer F.Cu) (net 13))
 (segment (start 43.434 24.914) (end 43.434 36.93019) (width 0.25) (layer F.Cu) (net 13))
 (segment (start 41.08 22.56) (end 43.434 24.914) (width 0.25) (layer F.Cu) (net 13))
 (segment (start 63.190999 38.606503) (end 61.047501 40.750001) (width 0.25) (layer F.Cu) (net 13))
 (segment (start 63.190999 36.250001) (end 63.190999 38.606503) (width 0.25) (layer F.Cu) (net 13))
 (segment (start 64.516 34.925) (end 63.190999 36.250001) (width 0.25) (layer F.Cu) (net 13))
 (segment (start 64.516 34.925) (end 71.016 34.925) (width 0.25) (layer F.Cu) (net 13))
 (segment (start 21.418801 22.904199) (end 20.2438 24.0792) (width 0.25) (layer B.Cu) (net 11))
 (segment (start 29.015 24.12) (end 27.849999 22.954999) (width 0.25) (layer B.Cu) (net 11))
 (segment (start 27.799199 22.904199) (end 27.849999 22.954999) (width 0.25) (layer B.Cu) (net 11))
 (segment (start 21.418801 22.904199) (end 27.799199 22.904199) (width 0.25) (layer B.Cu) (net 11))
 (segment (start 30.190001 22.944999) (end 38.738901 22.944999) (width 0.25) (layer B.Cu) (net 11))
 (segment (start 29.015 24.12) (end 30.190001 22.944999) (width 0.25) (layer B.Cu) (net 11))
 (segment (start 41.08 20.6039) (end 41.08 18.3) (width 0.25) (layer B.Cu) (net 11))
 (segment (start 38.738901 22.944999) (end 41.08 20.6039) (width 0.25) (layer B.Cu) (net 11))
 (segment (start 53.4628 39.425) (end 52.587809 40.299991) (width 0.25) (layer F.Cu) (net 11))
 (segment (start 53.9115 39.425) (end 53.4628 39.425) (width 0.25) (layer F.Cu) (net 11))
 (segment (start 52.587809 40.299991) (end 47.440211 40.299991) (width 0.25) (layer F.Cu) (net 11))
 (segment (start 43.88401 21.10401) (end 41.08 18.3) (width 0.25) (layer F.Cu) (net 11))
 (segment (start 43.88401 36.74379) (end 43.88401 21.10401) (width 0.25) (layer F.Cu) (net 11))
 (segment (start 47.440211 40.299991) (end 43.88401 36.74379) (width 0.25) (layer F.Cu) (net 11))
 (segment (start 53.9115 39.425) (end 60.4115 39.425) (width 0.25) (layer F.Cu) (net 11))
 (segment (start 40.9575 24.5745) (end 40.687009 24.844991) (width 0.25) (layer B.Cu) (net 14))
 (segment (start 40.824991 24.844991) (end 41.08 25.1) (width 0.25) (layer B.Cu) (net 14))
 (segment (start 31.555 21.58) (end 31.76 21.58) (width 0.25) (layer B.Cu) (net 14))
 (segment (start 30.379999 22.755001) (end 31.555 21.58) (width 0.25) (layer F.Cu) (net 14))
 (segment (start 23.999601 22.755001) (end 30.379999 22.755001) (width 0.25) (layer F.Cu) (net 14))
 (segment (start 22.7838 21.5392) (end 23.999601 22.755001) (width 0.25) (layer F.Cu) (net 14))
 (segment (start 32.035 21.1) (end 31.555 21.58) (width 0.25) (layer B.Cu) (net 14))
 (segment (start 42.982521 36.017479) (end 42.98399 36.01601) (width 0.25) (layer F.Cu) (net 14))
 (segment (start 42.982521 36.139933) (end 42.982521 36.017479) (width 0.25) (layer F.Cu) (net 14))
 (segment (start 34.49659 25.1) (end 41.08 25.1) (width 0.25) (layer F.Cu) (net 14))
 (segment (start 31.555 22.15841) (end 34.49659 25.1) (width 0.25) (layer F.Cu) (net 14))
 (segment (start 31.555 21.58) (end 31.555 22.15841) (width 0.25) (layer F.Cu) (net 14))
 (segment (start 62.740989 41.200011) (end 64.516 39.425) (width 0.25) (layer F.Cu) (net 14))
 (segment (start 47.067411 41.200011) (end 62.740989 41.200011) (width 0.25) (layer F.Cu) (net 14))
 (segment (start 42.98399 37.11659) (end 47.067411 41.200011) (width 0.25) (layer F.Cu) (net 14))
 (segment (start 42.98399 27.00399) (end 42.98399 37.11659) (width 0.25) (layer F.Cu) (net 14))
 (segment (start 41.08 25.1) (end 42.98399 27.00399) (width 0.25) (layer F.Cu) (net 14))
 (segment (start 64.516 39.425) (end 71.016 39.425) (width 0.25) (layer F.Cu) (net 14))
 (segment (start 21.418801 20.364199) (end 20.2438 21.5392) (width 0.25) (layer B.Cu) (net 9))
 (segment (start 29.015 21.58) (end 27.849999 20.414999) (width 0.25) (layer B.Cu) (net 9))
 (segment (start 27.799199 20.364199) (end 27.849999 20.414999) (width 0.25) (layer B.Cu) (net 9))
 (segment (start 21.418801 20.364199) (end 27.799199 20.364199) (width 0.25) (layer B.Cu) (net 9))
 (segment (start 29.015 21.58) (end 30.379999 20.215001) (width 0.25) (layer B.Cu) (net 9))
 (segment (start 36.624999 20.215001) (end 30.379999 20.215001) (width 0.25) (layer B.Cu) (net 9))
 (segment (start 41.08 15.76) (end 36.624999 20.215001) (width 0.25) (layer B.Cu) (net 9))
 (segment (start 51.525517 39.849981) (end 47.626611 39.849981) (width 0.25) (layer F.Cu) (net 9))
 (segment (start 47.626611 39.849981) (end 44.33402 36.55739) (width 0.25) (layer F.Cu) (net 9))
 (segment (start 44.33402 19.01402) (end 41.08 15.76) (width 0.25) (layer F.Cu) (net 9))
 (segment (start 44.33402 36.55739) (end 44.33402 19.01402) (width 0.25) (layer F.Cu) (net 9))
 (segment (start 53.9115 37.463998) (end 51.525517 39.849981) (width 0.25) (layer F.Cu) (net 9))
 (segment (start 53.9115 34.925) (end 53.9115 37.463998) (width 0.25) (layer F.Cu) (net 9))
 (segment (start 53.9115 34.925) (end 60.4115 34.925) (width 0.25) (layer F.Cu) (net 9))
 (segment (start 65.584 31.242) (end 65.5955 31.2305) (width 0.25) (layer F.Cu) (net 10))
 (segment (start 70.6755 30.4165) (end 70.6755 25.0825) (width 0.25) (layer F.Cu) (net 10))
 (segment (start 69.8615 31.2305) (end 70.6755 30.4165) (width 0.25) (layer F.Cu) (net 10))
 (segment (start 66.1041 31.2305) (end 66.0908 31.2172) (width 0.25) (layer F.Cu) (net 10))
 (segment (start 69.8615 31.2305) (end 66.1041 31.2305) (width 0.25) (layer F.Cu) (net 10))
 (segment (start 66.066 31.242) (end 66.0908 31.2172) (width 0.25) (layer F.Cu) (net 10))
 (segment (start 62.0776 31.242) (end 66.066 31.242) (width 0.25) (layer F.Cu) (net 10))
 (segment (start 49.0055 16.0655) (end 48.7 15.76) (width 0.25) (layer F.Cu) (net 10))
 (segment (start 53.96019 16.0655) (end 49.0055 16.0655) (width 0.25) (layer F.Cu) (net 10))
 (segment (start 55.63701 17.74232) (end 53.96019 16.0655) (width 0.25) (layer F.Cu) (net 10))
 (segment (start 55.63701 19.5676) (end 55.63701 17.74232) (width 0.25) (layer F.Cu) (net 10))
 (segment (start 59.43741 23.368) (end 55.63701 19.5676) (width 0.25) (layer F.Cu) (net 10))
 (segment (start 68.961 23.368) (end 59.43741 23.368) (width 0.25) (layer F.Cu) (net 10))
 (segment (start 70.6755 25.0825) (end 68.961 23.368) (width 0.25) (layer F.Cu) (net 10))
 (segment (start 48.7 22.56) (end 47.574999 21.434999) (width 0.25) (layer F.Cu) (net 10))
 (segment (start 47.574999 21.434999) (end 47.574999 16.885001) (width 0.25) (layer F.Cu) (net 10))
 (segment (start 47.574999 16.885001) (end 48.7 15.76) (width 0.25) (layer F.Cu) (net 10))
 (segment (start 49.71219 30.24219) (end 48.72 29.25) (width 0.25) (layer F.Cu) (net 4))
 (segment (start 49.845001 34.874999) (end 48.72 36) (width 0.25) (layer F.Cu) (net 4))
 (segment (start 49.845001 30.375001) (end 49.845001 34.874999) (width 0.25) (layer F.Cu) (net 4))
 (segment (start 49.71219 30.24219) (end 49.845001 30.375001) (width 0.25) (layer F.Cu) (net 4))
 (segment (start 68.1355 25.0825) (end 68.1355 29.2645) (width 0.25) (layer F.Cu) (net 4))
 (segment (start 68.1355 29.2645) (end 67.8 29.6) (width 0.25) (layer F.Cu) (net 4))
 (segment (start 50.620002 29.6) (end 49.845001 30.375001) (width 0.25) (layer F.Cu) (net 4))
 (segment (start 67.8 29.6) (end 50.620002 29.6) (width 0.25) (layer F.Cu) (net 4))
 (segment (start 66.0908 25.5778) (end 65.5955 25.0825) (width 0.25) (layer F.Cu) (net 2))
 (segment (start 66.0908 28.1172) (end 66.0908 25.5778) (width 0.25) (layer F.Cu) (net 2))
 (segment (start 50.8 36.46) (end 48.72 38.54) (width 0.25) (layer B.Cu) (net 2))
 (segment (start 50.8 34) (end 50.8 36.46) (width 0.25) (layer B.Cu) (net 2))
 (segment (start 52.55999 32.24001) (end 50.8 34) (width 0.25) (layer B.Cu) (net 2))
 (segment (start 59.8964 32.24001) (end 52.55999 32.24001) (width 0.25) (layer B.Cu) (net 2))
 (segment (start 65.5955 26.54091) (end 59.8964 32.24001) (width 0.25) (layer B.Cu) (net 2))
 (segment (start 65.5955 25.0825) (end 65.5955 26.54091) (width 0.25) (layer B.Cu) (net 2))
 (segment (start 62.992 25.146) (end 63.0555 25.0825) (width 0.25) (layer F.Cu) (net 6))
 (segment (start 63.0555 27.1641) (end 62.0776 28.142) (width 0.25) (layer F.Cu) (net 6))
 (segment (start 63.0555 25.0825) (end 63.0555 27.1641) (width 0.25) (layer F.Cu) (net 6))
 (segment (start 62.0776 28.142) (end 62.0776 28.66108) (width 0.25) (layer F.Cu) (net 6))
 (segment (start 48.72 31.79) (end 59.71 31.79) (width 0.25) (layer B.Cu) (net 6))
 (segment (start 63.0555 28.4445) (end 63.0555 25.0825) (width 0.25) (layer B.Cu) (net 6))
 (segment (start 59.71 31.79) (end 63.0555 28.4445) (width 0.25) (layer B.Cu) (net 6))
 (segment (start 54.662 19.229) (end 60.5155 25.0825) (width 0.25) (layer F.Cu) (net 15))
 (segment (start 54.662 18.6055) (end 54.662 19.229) (width 0.25) (layer F.Cu) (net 15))
 (segment (start 54.6868 22.2758) (end 56.8706 22.2758) (width 0.25) (layer F.Cu) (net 16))
 (segment (start 57.9755 23.3807) (end 57.9755 25.0825) (width 0.25) (layer F.Cu) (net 16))
 (segment (start 56.8706 22.2758) (end 57.9755 23.3807) (width 0.25) (layer F.Cu) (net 16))
 (segment (start 51.5242 22.2758) (end 48.7 25.1) (width 0.25) (layer F.Cu) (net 12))
 (segment (start 51.5868 22.2758) (end 51.5242 22.2758) (width 0.25) (layer F.Cu) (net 12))
 (segment (start 49.0055 18.6055) (end 48.7 18.3) (width 0.25) (layer F.Cu) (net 8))
 (segment (start 51.562 18.6055) (end 49.0055 18.6055) (width 0.25) (layer F.Cu) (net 8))
 (segment (start 23.968801 17.814199) (end 22.7838 18.9992) (width 0.25) (layer F.Cu) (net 21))
 (segment (start 31.555 19.04) (end 30.379999 17.864999) (width 0.25) (layer F.Cu) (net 21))
 (segment (start 34.27081 23.55201) (end 35.82568 23.55201) (width 0.25) (layer F.Cu) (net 21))
 (segment (start 33.180011 22.461211) (end 34.27081 23.55201) (width 0.25) (layer F.Cu) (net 21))
 (segment (start 33.180011 20.665011) (end 33.180011 22.461211) (width 0.25) (layer F.Cu) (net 21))
 (segment (start 31.555 19.04) (end 33.180011 20.665011) (width 0.25) (layer F.Cu) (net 21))
 (segment (start 30.329199 17.814199) (end 30.379999 17.864999) (width 0.25) (layer F.Cu) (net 21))
 (segment (start 23.968801 17.814199) (end 30.329199 17.814199) (width 0.25) (layer F.Cu) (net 21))
 (segment (start 34.998 15.8115) (end 35.5981 15.8115) (width 0.25) (layer F.Cu) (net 21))
 (segment (start 35.5981 15.8115) (end 36.703 16.9164) (width 0.25) (layer F.Cu) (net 21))
 (segment (start 36.703 22.67469) (end 35.82568 23.55201) (width 0.25) (layer F.Cu) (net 21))
 (segment (start 36.703 16.9164) (end 36.703 22.67469) (width 0.25) (layer F.Cu) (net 21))
 (segment (start 22.7838 16.4592) (end 23.968801 15.274199) (width 0.25) (layer F.Cu) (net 22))
 (segment (start 30.379999 15.324999) (end 31.555 16.5) (width 0.25) (layer F.Cu) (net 22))
 (segment (start 36.77299 14.61149) (end 37.973 15.8115) (width 0.25) (layer F.Cu) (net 22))
 (segment (start 33.44351 14.61149) (end 36.77299 14.61149) (width 0.25) (layer F.Cu) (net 22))
 (segment (start 31.555 16.5) (end 33.44351 14.61149) (width 0.25) (layer F.Cu) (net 22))
 (segment (start 30.329199 15.274199) (end 30.379999 15.324999) (width 0.25) (layer F.Cu) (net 22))
 (segment (start 23.968801 15.274199) (end 30.329199 15.274199) (width 0.25) (layer F.Cu) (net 22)))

